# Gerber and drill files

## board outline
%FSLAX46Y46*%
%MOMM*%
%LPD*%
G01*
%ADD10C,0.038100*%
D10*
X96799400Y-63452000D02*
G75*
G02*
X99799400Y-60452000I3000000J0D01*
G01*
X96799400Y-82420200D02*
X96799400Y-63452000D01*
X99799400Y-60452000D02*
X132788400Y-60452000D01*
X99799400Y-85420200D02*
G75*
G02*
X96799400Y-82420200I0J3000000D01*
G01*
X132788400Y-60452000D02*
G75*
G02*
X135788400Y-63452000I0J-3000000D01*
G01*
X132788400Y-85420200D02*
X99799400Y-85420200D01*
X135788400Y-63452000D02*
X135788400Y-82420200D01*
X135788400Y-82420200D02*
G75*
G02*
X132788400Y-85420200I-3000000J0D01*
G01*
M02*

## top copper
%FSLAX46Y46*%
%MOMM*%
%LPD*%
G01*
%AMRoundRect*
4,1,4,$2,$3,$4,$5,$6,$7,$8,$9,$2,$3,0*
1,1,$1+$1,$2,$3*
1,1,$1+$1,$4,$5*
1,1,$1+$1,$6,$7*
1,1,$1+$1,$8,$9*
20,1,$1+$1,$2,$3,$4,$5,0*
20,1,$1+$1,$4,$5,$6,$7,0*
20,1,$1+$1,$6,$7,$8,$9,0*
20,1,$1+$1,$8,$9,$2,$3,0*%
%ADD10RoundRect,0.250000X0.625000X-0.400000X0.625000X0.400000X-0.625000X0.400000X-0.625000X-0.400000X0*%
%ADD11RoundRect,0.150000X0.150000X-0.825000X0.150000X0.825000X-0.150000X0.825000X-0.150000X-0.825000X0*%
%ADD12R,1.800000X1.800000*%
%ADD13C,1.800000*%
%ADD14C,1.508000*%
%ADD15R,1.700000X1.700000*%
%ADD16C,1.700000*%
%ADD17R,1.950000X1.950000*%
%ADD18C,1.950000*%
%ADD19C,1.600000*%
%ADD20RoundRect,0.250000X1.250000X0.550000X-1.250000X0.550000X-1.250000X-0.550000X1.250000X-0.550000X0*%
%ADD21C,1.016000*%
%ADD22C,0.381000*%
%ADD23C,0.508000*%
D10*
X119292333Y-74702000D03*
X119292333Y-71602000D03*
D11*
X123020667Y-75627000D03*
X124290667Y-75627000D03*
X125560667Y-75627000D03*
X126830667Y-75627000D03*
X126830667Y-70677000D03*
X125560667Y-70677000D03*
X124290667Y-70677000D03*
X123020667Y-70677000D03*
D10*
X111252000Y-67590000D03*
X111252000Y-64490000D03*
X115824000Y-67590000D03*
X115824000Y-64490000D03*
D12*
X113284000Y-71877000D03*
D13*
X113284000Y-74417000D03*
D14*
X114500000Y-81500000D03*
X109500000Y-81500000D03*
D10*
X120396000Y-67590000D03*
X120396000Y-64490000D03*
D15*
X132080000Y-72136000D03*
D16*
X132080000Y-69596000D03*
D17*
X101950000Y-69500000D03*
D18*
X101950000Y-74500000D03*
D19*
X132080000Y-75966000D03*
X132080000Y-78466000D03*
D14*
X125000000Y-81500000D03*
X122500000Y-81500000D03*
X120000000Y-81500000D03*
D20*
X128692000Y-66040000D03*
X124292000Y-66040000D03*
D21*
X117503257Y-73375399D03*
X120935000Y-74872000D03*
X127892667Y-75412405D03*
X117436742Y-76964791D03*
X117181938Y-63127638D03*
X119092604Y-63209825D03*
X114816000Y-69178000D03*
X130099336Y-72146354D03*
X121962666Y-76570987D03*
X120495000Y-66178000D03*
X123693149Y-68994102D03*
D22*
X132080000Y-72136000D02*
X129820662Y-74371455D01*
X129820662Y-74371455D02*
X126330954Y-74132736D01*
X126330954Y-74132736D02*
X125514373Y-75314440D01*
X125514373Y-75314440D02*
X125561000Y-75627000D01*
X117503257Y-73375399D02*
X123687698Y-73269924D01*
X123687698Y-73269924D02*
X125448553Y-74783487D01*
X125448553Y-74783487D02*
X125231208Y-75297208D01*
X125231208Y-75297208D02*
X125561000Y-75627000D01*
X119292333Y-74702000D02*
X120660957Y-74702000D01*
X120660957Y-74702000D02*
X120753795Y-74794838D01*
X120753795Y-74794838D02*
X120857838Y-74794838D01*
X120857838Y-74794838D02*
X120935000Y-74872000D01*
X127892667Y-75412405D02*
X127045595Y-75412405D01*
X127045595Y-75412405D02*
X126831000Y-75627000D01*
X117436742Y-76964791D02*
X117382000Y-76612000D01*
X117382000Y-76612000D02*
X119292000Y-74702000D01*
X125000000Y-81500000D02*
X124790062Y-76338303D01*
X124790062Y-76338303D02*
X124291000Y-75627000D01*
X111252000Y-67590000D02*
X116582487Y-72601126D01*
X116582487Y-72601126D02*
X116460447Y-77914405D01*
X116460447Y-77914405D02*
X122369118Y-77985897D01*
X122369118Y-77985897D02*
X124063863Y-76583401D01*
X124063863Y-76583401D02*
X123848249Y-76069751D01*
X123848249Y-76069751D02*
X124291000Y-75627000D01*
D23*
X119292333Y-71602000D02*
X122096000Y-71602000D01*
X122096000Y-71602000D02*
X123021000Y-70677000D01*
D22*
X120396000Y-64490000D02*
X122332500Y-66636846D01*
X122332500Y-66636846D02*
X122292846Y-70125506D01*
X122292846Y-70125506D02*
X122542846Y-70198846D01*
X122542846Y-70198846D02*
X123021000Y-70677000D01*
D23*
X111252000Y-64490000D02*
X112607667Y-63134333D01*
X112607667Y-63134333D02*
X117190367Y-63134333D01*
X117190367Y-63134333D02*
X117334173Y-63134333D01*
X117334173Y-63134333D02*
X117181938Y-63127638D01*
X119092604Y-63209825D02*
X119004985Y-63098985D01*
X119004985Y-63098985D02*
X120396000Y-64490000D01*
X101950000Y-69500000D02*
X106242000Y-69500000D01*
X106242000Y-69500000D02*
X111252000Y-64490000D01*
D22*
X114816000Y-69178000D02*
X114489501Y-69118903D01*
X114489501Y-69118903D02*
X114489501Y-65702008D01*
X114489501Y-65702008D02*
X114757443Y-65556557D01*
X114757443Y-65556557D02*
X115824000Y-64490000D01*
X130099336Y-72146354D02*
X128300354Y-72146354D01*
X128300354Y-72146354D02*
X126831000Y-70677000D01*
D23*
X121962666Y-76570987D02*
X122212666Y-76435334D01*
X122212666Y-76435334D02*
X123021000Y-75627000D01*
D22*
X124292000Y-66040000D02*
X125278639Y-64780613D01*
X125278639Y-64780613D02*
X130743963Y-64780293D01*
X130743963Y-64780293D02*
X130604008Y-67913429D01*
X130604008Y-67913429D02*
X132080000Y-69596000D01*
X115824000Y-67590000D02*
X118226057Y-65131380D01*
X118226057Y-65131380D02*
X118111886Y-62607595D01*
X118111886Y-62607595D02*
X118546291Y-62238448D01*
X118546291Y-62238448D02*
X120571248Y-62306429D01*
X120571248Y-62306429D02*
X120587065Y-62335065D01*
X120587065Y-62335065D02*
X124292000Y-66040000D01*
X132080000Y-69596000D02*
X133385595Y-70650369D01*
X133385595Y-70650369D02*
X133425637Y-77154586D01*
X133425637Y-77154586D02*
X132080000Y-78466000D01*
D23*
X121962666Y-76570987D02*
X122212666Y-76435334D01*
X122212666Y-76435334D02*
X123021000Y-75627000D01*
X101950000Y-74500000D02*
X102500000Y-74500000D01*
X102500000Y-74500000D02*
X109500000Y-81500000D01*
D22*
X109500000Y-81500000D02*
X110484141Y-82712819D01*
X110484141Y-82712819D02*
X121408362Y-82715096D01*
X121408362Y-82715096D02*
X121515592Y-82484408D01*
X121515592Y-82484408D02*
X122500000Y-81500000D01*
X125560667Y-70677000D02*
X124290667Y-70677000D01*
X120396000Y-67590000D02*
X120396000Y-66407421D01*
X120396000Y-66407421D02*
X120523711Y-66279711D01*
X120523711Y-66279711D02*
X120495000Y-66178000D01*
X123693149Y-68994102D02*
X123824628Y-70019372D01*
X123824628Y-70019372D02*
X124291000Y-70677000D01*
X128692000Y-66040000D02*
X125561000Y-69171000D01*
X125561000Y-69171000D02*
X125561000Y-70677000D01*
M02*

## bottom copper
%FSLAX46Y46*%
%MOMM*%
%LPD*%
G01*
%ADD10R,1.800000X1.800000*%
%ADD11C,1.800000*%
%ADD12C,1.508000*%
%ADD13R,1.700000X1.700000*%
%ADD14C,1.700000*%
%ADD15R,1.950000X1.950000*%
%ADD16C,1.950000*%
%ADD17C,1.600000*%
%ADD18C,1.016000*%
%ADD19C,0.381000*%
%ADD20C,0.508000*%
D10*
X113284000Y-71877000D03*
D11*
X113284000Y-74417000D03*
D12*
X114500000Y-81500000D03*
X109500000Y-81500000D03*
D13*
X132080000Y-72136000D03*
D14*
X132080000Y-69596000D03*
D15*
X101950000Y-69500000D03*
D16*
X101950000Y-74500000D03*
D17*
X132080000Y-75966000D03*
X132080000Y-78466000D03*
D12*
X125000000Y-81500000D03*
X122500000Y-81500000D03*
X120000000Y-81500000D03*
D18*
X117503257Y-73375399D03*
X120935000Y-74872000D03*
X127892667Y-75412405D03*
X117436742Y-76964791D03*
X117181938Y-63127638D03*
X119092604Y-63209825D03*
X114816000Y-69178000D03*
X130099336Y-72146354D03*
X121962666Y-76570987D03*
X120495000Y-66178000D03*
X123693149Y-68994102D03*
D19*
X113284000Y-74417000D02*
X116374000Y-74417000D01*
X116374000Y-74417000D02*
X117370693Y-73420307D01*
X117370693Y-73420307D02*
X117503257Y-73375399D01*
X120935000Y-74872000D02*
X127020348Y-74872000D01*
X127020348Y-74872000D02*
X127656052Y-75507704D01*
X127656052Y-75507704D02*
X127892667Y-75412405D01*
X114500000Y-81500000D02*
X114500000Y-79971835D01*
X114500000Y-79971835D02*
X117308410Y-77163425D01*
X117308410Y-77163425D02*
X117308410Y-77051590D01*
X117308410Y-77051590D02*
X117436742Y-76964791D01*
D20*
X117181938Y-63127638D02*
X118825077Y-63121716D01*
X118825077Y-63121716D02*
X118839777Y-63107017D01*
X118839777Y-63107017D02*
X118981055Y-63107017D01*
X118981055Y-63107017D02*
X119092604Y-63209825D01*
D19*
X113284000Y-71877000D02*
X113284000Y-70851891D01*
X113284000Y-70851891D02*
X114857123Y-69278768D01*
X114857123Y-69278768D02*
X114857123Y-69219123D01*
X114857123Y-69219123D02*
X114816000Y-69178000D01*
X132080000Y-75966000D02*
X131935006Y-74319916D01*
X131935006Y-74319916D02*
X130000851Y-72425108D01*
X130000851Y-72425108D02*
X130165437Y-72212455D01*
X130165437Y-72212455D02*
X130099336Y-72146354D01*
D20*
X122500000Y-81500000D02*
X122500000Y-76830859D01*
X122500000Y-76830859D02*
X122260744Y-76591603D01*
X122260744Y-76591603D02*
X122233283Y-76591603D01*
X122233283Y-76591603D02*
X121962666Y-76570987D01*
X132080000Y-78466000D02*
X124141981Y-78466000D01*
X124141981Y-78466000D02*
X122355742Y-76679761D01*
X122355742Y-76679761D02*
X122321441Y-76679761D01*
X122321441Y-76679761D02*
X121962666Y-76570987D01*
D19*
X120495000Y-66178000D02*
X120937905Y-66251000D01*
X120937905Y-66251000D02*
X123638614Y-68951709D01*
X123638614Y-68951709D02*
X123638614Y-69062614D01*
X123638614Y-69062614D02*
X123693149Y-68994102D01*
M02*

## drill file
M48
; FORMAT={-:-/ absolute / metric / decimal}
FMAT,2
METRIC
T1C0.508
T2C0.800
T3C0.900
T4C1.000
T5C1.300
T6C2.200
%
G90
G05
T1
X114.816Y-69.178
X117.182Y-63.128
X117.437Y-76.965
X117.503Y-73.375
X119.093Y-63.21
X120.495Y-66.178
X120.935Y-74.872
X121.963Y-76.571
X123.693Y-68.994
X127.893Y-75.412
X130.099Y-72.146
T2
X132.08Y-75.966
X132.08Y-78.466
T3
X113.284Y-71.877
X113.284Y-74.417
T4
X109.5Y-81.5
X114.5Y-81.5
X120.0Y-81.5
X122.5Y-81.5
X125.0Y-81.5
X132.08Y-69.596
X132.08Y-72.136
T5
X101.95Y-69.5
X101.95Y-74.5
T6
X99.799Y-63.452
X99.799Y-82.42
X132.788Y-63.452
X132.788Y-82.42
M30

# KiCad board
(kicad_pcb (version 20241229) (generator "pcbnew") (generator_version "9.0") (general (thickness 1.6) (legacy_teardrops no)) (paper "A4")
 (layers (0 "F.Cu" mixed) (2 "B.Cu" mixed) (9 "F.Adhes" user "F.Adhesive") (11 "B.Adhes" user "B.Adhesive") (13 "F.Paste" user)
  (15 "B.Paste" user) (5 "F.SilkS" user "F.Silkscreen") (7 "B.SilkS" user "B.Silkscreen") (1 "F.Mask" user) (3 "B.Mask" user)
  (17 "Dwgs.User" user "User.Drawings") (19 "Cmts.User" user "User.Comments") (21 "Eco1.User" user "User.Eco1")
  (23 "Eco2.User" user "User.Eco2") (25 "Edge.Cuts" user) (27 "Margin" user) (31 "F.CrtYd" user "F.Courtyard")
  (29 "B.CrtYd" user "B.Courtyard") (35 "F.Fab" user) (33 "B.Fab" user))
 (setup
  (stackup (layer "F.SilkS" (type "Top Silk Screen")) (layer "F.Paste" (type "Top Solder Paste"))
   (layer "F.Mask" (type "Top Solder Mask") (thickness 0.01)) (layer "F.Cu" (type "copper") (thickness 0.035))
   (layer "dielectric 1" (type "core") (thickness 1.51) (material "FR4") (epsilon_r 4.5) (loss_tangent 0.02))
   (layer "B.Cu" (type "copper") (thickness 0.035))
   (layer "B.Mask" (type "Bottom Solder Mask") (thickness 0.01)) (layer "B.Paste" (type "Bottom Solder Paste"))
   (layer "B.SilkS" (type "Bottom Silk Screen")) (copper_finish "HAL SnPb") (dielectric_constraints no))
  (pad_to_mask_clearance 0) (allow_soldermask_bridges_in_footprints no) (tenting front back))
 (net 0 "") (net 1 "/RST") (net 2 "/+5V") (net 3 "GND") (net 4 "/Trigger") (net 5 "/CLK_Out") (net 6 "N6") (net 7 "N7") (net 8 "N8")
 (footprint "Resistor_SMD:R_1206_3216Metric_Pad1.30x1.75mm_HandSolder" (layer "F.Cu") (at 119.292333 73.152 90)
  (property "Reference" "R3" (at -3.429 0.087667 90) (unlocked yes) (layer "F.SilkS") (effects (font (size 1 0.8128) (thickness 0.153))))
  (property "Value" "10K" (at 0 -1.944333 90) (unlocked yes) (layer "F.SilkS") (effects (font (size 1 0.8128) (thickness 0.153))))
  (pad "1" smd roundrect (at -1.55 0 90) (size 1.3 1.75) (layers "F.Cu" "F.Mask" "F.Paste") (roundrect_rratio 0.192308) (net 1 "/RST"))
  (pad "2" smd roundrect (at 1.55 0 90) (size 1.3 1.75) (layers "F.Cu" "F.Mask" "F.Paste") (roundrect_rratio 0.192308) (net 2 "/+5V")))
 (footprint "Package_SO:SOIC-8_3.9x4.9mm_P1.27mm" (layer "F.Cu") (at 124.925667 73.152 90)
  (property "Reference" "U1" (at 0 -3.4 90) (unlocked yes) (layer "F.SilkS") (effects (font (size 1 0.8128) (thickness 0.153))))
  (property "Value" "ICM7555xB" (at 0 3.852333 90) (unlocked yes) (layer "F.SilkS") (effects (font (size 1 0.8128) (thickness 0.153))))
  (pad "1" smd roundrect (at -2.475 -1.905 90) (size 1.95 0.6) (layers "F.Cu" "F.Mask" "F.Paste") (roundrect_rratio 0.25) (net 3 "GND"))
  (pad "2" smd roundrect (at -2.475 -0.635 90) (size 1.95 0.6) (layers "F.Cu" "F.Mask" "F.Paste") (roundrect_rratio 0.25) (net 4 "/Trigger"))
  (pad "3" smd roundrect (at -2.475 0.635 90) (size 1.95 0.6) (layers "F.Cu" "F.Mask" "F.Paste") (roundrect_rratio 0.25) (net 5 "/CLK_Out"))
  (pad "4" smd roundrect (at -2.475 1.905 90) (size 1.95 0.6) (layers "F.Cu" "F.Mask" "F.Paste") (roundrect_rratio 0.25) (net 1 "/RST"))
  (pad "5" smd roundrect (at 2.475 1.905 90) (size 1.95 0.6) (layers "F.Cu" "F.Mask" "F.Paste") (roundrect_rratio 0.25) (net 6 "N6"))
  (pad "6" smd roundrect (at 2.475 0.635 90) (size 1.95 0.6) (layers "F.Cu" "F.Mask" "F.Paste") (roundrect_rratio 0.25) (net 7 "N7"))
  (pad "7" smd roundrect (at 2.475 -0.635 90) (size 1.95 0.6) (layers "F.Cu" "F.Mask" "F.Paste") (roundrect_rratio 0.25) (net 7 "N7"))
  (pad "8" smd roundrect (at 2.475 -1.905 90) (size 1.95 0.6) (layers "F.Cu" "F.Mask" "F.Paste") (roundrect_rratio 0.25) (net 2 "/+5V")))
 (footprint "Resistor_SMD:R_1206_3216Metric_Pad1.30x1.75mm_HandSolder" (layer "F.Cu") (at 111.252 66.04 90)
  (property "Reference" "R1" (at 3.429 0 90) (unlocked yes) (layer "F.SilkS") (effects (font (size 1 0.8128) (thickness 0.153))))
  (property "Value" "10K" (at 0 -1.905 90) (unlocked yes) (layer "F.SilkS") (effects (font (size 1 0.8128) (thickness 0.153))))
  (pad "1" smd roundrect (at -1.55 0 90) (size 1.3 1.75) (layers "F.Cu" "F.Mask" "F.Paste") (roundrect_rratio 0.192308) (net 4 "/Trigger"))
  (pad "2" smd roundrect (at 1.55 0 90) (size 1.3 1.75) (layers "F.Cu" "F.Mask" "F.Paste") (roundrect_rratio 0.192308) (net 2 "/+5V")))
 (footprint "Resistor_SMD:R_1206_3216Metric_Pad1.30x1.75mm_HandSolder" (layer "F.Cu") (at 115.824 66.04 90)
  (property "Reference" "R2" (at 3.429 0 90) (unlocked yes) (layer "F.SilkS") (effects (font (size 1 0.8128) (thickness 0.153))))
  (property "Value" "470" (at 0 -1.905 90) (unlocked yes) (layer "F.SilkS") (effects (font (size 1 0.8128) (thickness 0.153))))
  (pad "1" smd roundrect (at -1.55 0 90) (size 1.3 1.75) (layers "F.Cu" "F.Mask" "F.Paste") (roundrect_rratio 0.192308) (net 3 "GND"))
  (pad "2" smd roundrect (at 1.55 0 90) (size 1.3 1.75) (layers "F.Cu" "F.Mask" "F.Paste") (roundrect_rratio 0.192308) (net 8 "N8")))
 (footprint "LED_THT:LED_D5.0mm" (layer "F.Cu") (at 113.284 71.877 -90)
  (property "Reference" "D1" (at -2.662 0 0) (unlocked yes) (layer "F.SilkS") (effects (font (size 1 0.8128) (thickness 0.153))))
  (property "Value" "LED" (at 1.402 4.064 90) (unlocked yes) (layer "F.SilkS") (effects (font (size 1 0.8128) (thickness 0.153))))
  (pad "1" thru_hole rect (at 0 0 270) (size 1.8 1.8) (drill 0.9) (layers "*.Cu" "*.Mask") (remove_unused_layers no) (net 8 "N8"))
  (pad "2" thru_hole circle (at 2.54 0 270) (size 1.8 1.8) (drill 0.9) (layers "*.Cu" "*.Mask") (remove_unused_layers no) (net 5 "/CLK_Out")))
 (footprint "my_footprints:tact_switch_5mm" (layer "F.Cu") (at 112 81.5 180)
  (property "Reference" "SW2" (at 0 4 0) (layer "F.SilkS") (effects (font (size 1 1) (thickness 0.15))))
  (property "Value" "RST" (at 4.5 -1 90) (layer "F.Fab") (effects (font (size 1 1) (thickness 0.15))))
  (pad "1" thru_hole circle (at -2.5 0 180) (size 1.508 1.508) (drill 1) (layers "*.Cu" "*.Mask") (remove_unused_layers no) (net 1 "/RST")
   (solder_mask_margin 0.102))
  (pad "2" thru_hole circle (at 2.5 0 180) (size 1.508 1.508) (drill 1) (layers "*.Cu" "*.Mask") (remove_unused_layers no) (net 3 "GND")
   (solder_mask_margin 0.102)))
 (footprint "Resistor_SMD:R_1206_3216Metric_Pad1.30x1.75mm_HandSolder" (layer "F.Cu") (at 120.396 66.04 90)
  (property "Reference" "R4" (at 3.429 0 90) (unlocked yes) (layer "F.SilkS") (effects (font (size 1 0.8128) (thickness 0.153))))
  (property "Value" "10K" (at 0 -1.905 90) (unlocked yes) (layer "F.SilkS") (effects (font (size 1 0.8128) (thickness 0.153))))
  (pad "1" smd roundrect (at -1.55 0 90) (size 1.3 1.75) (layers "F.Cu" "F.Mask" "F.Paste") (roundrect_rratio 0.192308) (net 7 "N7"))
  (pad "2" smd roundrect (at 1.55 0 90) (size 1.3 1.75) (layers "F.Cu" "F.Mask" "F.Paste") (roundrect_rratio 0.192308) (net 2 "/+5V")))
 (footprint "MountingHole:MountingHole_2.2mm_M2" (layer "F.Cu") (at 99.7994 63.452)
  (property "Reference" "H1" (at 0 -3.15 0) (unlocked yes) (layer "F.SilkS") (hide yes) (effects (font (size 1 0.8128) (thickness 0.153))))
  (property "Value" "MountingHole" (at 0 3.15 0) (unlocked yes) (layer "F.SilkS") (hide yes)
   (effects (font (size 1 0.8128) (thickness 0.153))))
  (pad "" np_thru_hole circle (at 0 0) (size 2.2 2.2) (drill 2.2) (layers "*.Cu" "*.Mask")))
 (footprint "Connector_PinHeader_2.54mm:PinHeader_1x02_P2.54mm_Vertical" (layer "F.Cu") (at 132.08 72.136 180)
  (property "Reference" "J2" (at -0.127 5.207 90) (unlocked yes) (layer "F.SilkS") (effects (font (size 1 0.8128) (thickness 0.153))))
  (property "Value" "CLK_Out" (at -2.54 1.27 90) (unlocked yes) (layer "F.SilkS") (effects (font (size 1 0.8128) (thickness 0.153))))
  (pad "1" thru_hole rect (at 0 0 180) (size 1.7 1.7) (drill 1) (layers "*.Cu" "*.Mask") (remove_unused_layers no) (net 5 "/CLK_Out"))
  (pad "2" thru_hole circle (at 0 2.54 180) (size 1.7 1.7) (drill 1) (layers "*.Cu" "*.Mask") (remove_unused_layers no) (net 3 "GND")))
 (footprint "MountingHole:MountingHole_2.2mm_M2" (layer "F.Cu") (at 132.7884 82.4202)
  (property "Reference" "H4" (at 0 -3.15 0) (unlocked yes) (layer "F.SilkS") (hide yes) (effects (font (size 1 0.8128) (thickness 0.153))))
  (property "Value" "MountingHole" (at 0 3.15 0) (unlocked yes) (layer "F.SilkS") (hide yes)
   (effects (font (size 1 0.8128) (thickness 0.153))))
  (pad "" np_thru_hole circle (at 0 0) (size 2.2 2.2) (drill 2.2) (layers "*.Cu" "*.Mask")))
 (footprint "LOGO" (layer "F.Cu") (at 105.5 63.5)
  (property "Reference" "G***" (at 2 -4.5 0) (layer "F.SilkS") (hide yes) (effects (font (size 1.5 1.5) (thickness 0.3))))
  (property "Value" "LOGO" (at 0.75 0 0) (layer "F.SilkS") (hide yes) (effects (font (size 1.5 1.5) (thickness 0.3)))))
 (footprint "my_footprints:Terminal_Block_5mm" (layer "F.Cu") (at 101.95 72 -90)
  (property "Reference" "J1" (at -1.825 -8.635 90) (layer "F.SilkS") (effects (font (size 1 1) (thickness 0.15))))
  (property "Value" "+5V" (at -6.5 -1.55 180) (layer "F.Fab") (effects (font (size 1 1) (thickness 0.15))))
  (pad "1" thru_hole rect (at -2.5 0 270) (size 1.95 1.95) (drill 1.3) (layers "*.Cu" "*.Mask") (remove_unused_layers no) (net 2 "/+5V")
   (solder_mask_margin 0.102))
  (pad "2" thru_hole circle (at 2.5 0 270) (size 1.95 1.95) (drill 1.3) (layers "*.Cu" "*.Mask") (remove_unused_layers no) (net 3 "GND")
   (solder_mask_margin 0.102)))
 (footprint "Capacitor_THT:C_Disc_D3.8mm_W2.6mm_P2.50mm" (layer "F.Cu") (at 132.08 75.966 -90)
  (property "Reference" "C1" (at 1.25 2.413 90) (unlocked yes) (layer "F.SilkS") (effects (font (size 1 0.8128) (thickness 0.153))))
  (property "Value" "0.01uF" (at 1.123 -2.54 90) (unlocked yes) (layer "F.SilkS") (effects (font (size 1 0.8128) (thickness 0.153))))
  (pad "1" thru_hole circle (at 0 0 270) (size 1.6 1.6) (drill 0.8) (layers "*.Cu" "*.Mask") (remove_unused_layers no) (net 6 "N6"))
  (pad "2" thru_hole circle (at 2.5 0 270) (size 1.6 1.6) (drill 0.8) (layers "*.Cu" "*.Mask") (remove_unused_layers no) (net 3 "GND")))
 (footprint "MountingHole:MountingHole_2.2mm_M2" (layer "F.Cu") (at 132.7884 63.452)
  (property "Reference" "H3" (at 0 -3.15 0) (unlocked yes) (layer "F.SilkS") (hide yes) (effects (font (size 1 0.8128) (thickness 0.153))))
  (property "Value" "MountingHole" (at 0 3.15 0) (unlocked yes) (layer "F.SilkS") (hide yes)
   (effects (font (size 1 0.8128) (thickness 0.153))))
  (pad "" np_thru_hole circle (at 0 0) (size 2.2 2.2) (drill 2.2) (layers "*.Cu" "*.Mask")))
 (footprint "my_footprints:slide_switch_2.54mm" (layer "F.Cu") (at 122.5 81.5 180)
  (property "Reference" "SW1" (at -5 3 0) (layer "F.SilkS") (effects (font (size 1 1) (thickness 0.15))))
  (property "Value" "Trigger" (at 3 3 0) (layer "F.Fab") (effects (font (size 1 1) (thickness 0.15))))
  (pad "1" thru_hole circle (at -2.5 0 180) (size 1.508 1.508) (drill 1) (layers "*.Cu" "*.Mask") (remove_unused_layers no)
   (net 4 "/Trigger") (solder_mask_margin 0.102))
  (pad "2" thru_hole circle (at 0 0 180) (size 1.508 1.508) (drill 1) (layers "*.Cu" "*.Mask") (remove_unused_layers no) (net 3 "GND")
   (solder_mask_margin 0.102))
  (pad "3" thru_hole circle (at 2.5 0 180) (size 1.508 1.508) (drill 1) (layers "*.Cu" "*.Mask") (remove_unused_layers no)
   (solder_mask_margin 0.102)))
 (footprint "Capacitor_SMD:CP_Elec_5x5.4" (layer "F.Cu") (at 126.492 66.04 180)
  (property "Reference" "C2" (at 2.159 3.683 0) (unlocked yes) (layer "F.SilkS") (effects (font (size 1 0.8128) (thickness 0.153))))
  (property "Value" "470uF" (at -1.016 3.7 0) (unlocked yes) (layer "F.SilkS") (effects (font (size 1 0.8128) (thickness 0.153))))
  (pad "1" smd roundrect (at -2.2 0 180) (size 3 1.6) (layers "F.Cu" "F.Mask" "F.Paste") (roundrect_rratio 0.15625) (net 7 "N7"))
  (pad "2" smd roundrect (at 2.2 0 180) (size 3 1.6) (layers "F.Cu" "F.Mask" "F.Paste") (roundrect_rratio 0.15625) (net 3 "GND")))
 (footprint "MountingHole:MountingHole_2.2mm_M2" (layer "F.Cu") (at 99.7994 82.4202)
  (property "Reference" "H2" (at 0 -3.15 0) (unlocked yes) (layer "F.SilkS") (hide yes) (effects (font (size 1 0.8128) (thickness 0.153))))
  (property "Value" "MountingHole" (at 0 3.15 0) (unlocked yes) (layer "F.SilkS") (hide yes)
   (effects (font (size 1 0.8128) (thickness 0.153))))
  (pad "" np_thru_hole circle (at 0 0) (size 2.2 2.2) (drill 2.2) (layers "*.Cu" "*.Mask")))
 (gr_arc (start 96.7994 63.452) (mid 97.67808 61.33068) (end 99.7994 60.452) (stroke (width 0.0381) (type default)) (layer "Edge.Cuts"))
 (gr_line (start 96.7994 82.4202) (end 96.7994 63.452) (stroke (width 0.0381) (type default)) (layer "Edge.Cuts"))
 (gr_line (start 99.7994 60.452) (end 132.7884 60.452) (stroke (width 0.0381) (type default)) (layer "Edge.Cuts"))
 (gr_arc (start 99.7994 85.4202) (mid 97.67808 84.54152) (end 96.7994 82.4202) (stroke (width 0.0381) (type default)) (layer "Edge.Cuts"))
 (gr_arc (start 132.7884 60.452) (mid 134.90972 61.33068) (end 135.7884 63.452) (stroke (width 0.0381) (type default)) (layer "Edge.Cuts"))
 (gr_line (start 132.7884 85.4202) (end 99.7994 85.4202) (stroke (width 0.0381) (type default)) (layer "Edge.Cuts"))
 (gr_line (start 135.7884 63.452) (end 135.7884 82.4202) (stroke (width 0.0381) (type default)) (layer "Edge.Cuts"))
 (gr_arc (start 135.7884 82.4202) (mid 134.90972 84.54152) (end 132.7884 85.4202) (stroke (width 0.0381) (type default)) (layer "Edge.Cuts"))
 (segment (start 132.080000 72.136000) (end 129.820662 74.371455) (width 0.381000) (layer "F.Cu") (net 5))
 (segment (start 129.820662 74.371455) (end 126.330954 74.132736) (width 0.381000) (layer "F.Cu") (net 5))
 (segment (start 126.330954 74.132736) (end 125.514373 75.314440) (width 0.381000) (layer "F.Cu") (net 5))
 (segment (start 125.514373 75.314440) (end 125.561000 75.627000) (width 0.381000) (layer "F.Cu") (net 5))
 (segment (start 113.284000 74.417000) (end 116.374000 74.417000) (width 0.381000) (layer "B.Cu") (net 5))
 (segment (start 116.374000 74.417000) (end 117.370693 73.420307) (width 0.381000) (layer "B.Cu") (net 5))
 (segment (start 117.370693 73.420307) (end 117.503257 73.375399) (width 0.381000) (layer "B.Cu") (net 5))
 (segment (start 117.503257 73.375399) (end 123.687698 73.269924) (width 0.381000) (layer "F.Cu") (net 5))
 (segment (start 123.687698 73.269924) (end 125.448553 74.783487) (width 0.381000) (layer "F.Cu") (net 5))
 (segment (start 125.448553 74.783487) (end 125.231208 75.297208) (width 0.381000) (layer "F.Cu") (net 5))
 (segment (start 125.231208 75.297208) (end 125.561000 75.627000) (width 0.381000) (layer "F.Cu") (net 5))
 (segment (start 119.292333 74.702000) (end 120.660957 74.702000) (width 0.381000) (layer "F.Cu") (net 1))
 (segment (start 120.660957 74.702000) (end 120.753795 74.794838) (width 0.381000) (layer "F.Cu") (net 1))
 (segment (start 120.753795 74.794838) (end 120.857838 74.794838) (width 0.381000) (layer "F.Cu") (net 1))
 (segment (start 120.857838 74.794838) (end 120.935000 74.872000) (width 0.381000) (layer "F.Cu") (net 1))
 (segment (start 120.935000 74.872000) (end 127.020348 74.872000) (width 0.381000) (layer "B.Cu") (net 1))
 (segment (start 127.020348 74.872000) (end 127.656052 75.507704) (width 0.381000) (layer "B.Cu") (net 1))
 (segment (start 127.656052 75.507704) (end 127.892667 75.412405) (width 0.381000) (layer "B.Cu") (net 1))
 (segment (start 127.892667 75.412405) (end 127.045595 75.412405) (width 0.381000) (layer "F.Cu") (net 1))
 (segment (start 127.045595 75.412405) (end 126.831000 75.627000) (width 0.381000) (layer "F.Cu") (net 1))
 (segment (start 114.500000 81.500000) (end 114.500000 79.971835) (width 0.381000) (layer "B.Cu") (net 1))
 (segment (start 114.500000 79.971835) (end 117.308410 77.163425) (width 0.381000) (layer "B.Cu") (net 1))
 (segment (start 117.308410 77.163425) (end 117.308410 77.051590) (width 0.381000) (layer "B.Cu") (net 1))
 (segment (start 117.308410 77.051590) (end 117.436742 76.964791) (width 0.381000) (layer "B.Cu") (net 1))
 (segment (start 117.436742 76.964791) (end 117.382000 76.612000) (width 0.381000) (layer "F.Cu") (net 1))
 (segment (start 117.382000 76.612000) (end 119.292000 74.702000) (width 0.381000) (layer "F.Cu") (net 1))
 (segment (start 125.000000 81.500000) (end 124.790062 76.338303) (width 0.381000) (layer "F.Cu") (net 4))
 (segment (start 124.790062 76.338303) (end 124.291000 75.627000) (width 0.381000) (layer "F.Cu") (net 4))
 (segment (start 111.252000 67.590000) (end 116.582487 72.601126) (width 0.381000) (layer "F.Cu") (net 4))
 (segment (start 116.582487 72.601126) (end 116.460447 77.914405) (width 0.381000) (layer "F.Cu") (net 4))
 (segment (start 116.460447 77.914405) (end 122.369118 77.985897) (width 0.381000) (layer "F.Cu") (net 4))
 (segment (start 122.369118 77.985897) (end 124.063863 76.583401) (width 0.381000) (layer "F.Cu") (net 4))
 (segment (start 124.063863 76.583401) (end 123.848249 76.069751) (width 0.381000) (layer "F.Cu") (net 4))
 (segment (start 123.848249 76.069751) (end 124.291000 75.627000) (width 0.381000) (layer "F.Cu") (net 4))
 (segment (start 119.292333 71.602000) (end 122.096000 71.602000) (width 0.508000) (layer "F.Cu") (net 2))
 (segment (start 122.096000 71.602000) (end 123.021000 70.677000) (width 0.508000) (layer "F.Cu") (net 2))
 (segment (start 120.396000 64.490000) (end 122.332500 66.636846) (width 0.381000) (layer "F.Cu") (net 2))
 (segment (start 122.332500 66.636846) (end 122.292846 70.125506) (width 0.381000) (layer "F.Cu") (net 2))
 (segment (start 122.292846 70.125506) (end 122.542846 70.198846) (width 0.381000) (layer "F.Cu") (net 2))
 (segment (start 122.542846 70.198846) (end 123.021000 70.677000) (width 0.381000) (layer "F.Cu") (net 2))
 (segment (start 111.252000 64.490000) (end 112.607667 63.134333) (width 0.508000) (layer "F.Cu") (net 2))
 (segment (start 112.607667 63.134333) (end 117.190367 63.134333) (width 0.508000) (layer "F.Cu") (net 2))
 (segment (start 117.190367 63.134333) (end 117.334173 63.134333) (width 0.508000) (layer "F.Cu") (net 2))
 (segment (start 117.334173 63.134333) (end 117.181938 63.127638) (width 0.508000) (layer "F.Cu") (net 2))
 (segment (start 117.181938 63.127638) (end 118.825077 63.121716) (width 0.508000) (layer "B.Cu") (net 2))
 (segment (start 118.825077 63.121716) (end 118.839777 63.107017) (width 0.508000) (layer "B.Cu") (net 2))
 (segment (start 118.839777 63.107017) (end 118.981055 63.107017) (width 0.508000) (layer "B.Cu") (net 2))
 (segment (start 118.981055 63.107017) (end 119.092604 63.209825) (width 0.508000) (layer "B.Cu") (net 2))
 (segment (start 119.092604 63.209825) (end 119.004985 63.098985) (width 0.508000) (layer "F.Cu") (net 2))
 (segment (start 119.004985 63.098985) (end 120.396000 64.490000) (width 0.508000) (layer "F.Cu") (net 2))
 (segment (start 101.950000 69.500000) (end 106.242000 69.500000) (width 0.508000) (layer "F.Cu") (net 2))
 (segment (start 106.242000 69.500000) (end 111.252000 64.490000) (width 0.508000) (layer "F.Cu") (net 2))
 (segment (start 113.284000 71.877000) (end 113.284000 70.851891) (width 0.381000) (layer "B.Cu") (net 8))
 (segment (start 113.284000 70.851891) (end 114.857123 69.278768) (width 0.381000) (layer "B.Cu") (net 8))
 (segment (start 114.857123 69.278768) (end 114.857123 69.219123) (width 0.381000) (layer "B.Cu") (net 8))
 (segment (start 114.857123 69.219123) (end 114.816000 69.178000) (width 0.381000) (layer "B.Cu") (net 8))
 (segment (start 114.816000 69.178000) (end 114.489501 69.118903) (width 0.381000) (layer "F.Cu") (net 8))
 (segment (start 114.489501 69.118903) (end 114.489501 65.702008) (width 0.381000) (layer "F.Cu") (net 8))
 (segment (start 114.489501 65.702008) (end 114.757443 65.556557) (width 0.381000) (layer "F.Cu") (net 8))
 (segment (start 114.757443 65.556557) (end 115.824000 64.490000) (width 0.381000) (layer "F.Cu") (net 8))
 (segment (start 132.080000 75.966000) (end 131.935006 74.319916) (width 0.381000) (layer "B.Cu") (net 6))
 (segment (start 131.935006 74.319916) (end 130.000851 72.425108) (width 0.381000) (layer "B.Cu") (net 6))
 (segment (start 130.000851 72.425108) (end 130.165437 72.212455) (width 0.381000) (layer "B.Cu") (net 6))
 (segment (start 130.165437 72.212455) (end 130.099336 72.146354) (width 0.381000) (layer "B.Cu") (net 6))
 (segment (start 130.099336 72.146354) (end 128.300354 72.146354) (width 0.381000) (layer "F.Cu") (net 6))
 (segment (start 128.300354 72.146354) (end 126.831000 70.677000) (width 0.381000) (layer "F.Cu") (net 6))
 (segment (start 122.500000 81.500000) (end 122.500000 76.830859) (width 0.508000) (layer "B.Cu") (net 3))
 (segment (start 122.500000 76.830859) (end 122.260744 76.591603) (width 0.508000) (layer "B.Cu") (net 3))
 (segment (start 122.260744 76.591603) (end 122.233283 76.591603) (width 0.508000) (layer "B.Cu") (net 3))
 (segment (start 122.233283 76.591603) (end 121.962666 76.570987) (width 0.508000) (layer "B.Cu") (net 3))
 (segment (start 121.962666 76.570987) (end 122.212666 76.435334) (width 0.508000) (layer "F.Cu") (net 3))
 (segment (start 122.212666 76.435334) (end 123.021000 75.627000) (width 0.508000) (layer "F.Cu") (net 3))
 (segment (start 124.292000 66.040000) (end 125.278639 64.780613) (width 0.381000) (layer "F.Cu") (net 3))
 (segment (start 125.278639 64.780613) (end 130.743963 64.780293) (width 0.381000) (layer "F.Cu") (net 3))
 (segment (start 130.743963 64.780293) (end 130.604008 67.913429) (width 0.381000) (layer "F.Cu") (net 3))
 (segment (start 130.604008 67.913429) (end 132.080000 69.596000) (width 0.381000) (layer "F.Cu") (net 3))
 (segment (start 115.824000 67.590000) (end 118.226057 65.131380) (width 0.381000) (layer "F.Cu") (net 3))
 (segment (start 118.226057 65.131380) (end 118.111886 62.607595) (width 0.381000) (layer "F.Cu") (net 3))
 (segment (start 118.111886 62.607595) (end 118.546291 62.238448) (width 0.381000) (layer "F.Cu") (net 3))
 (segment (start 118.546291 62.238448) (end 120.571248 62.306429) (width 0.381000) (layer "F.Cu") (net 3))
 (segment (start 120.571248 62.306429) (end 120.587065 62.335065) (width 0.381000) (layer "F.Cu") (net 3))
 (segment (start 120.587065 62.335065) (end 124.292000 66.040000) (width 0.381000) (layer "F.Cu") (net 3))
 (segment (start 132.080000 69.596000) (end 133.385595 70.650369) (width 0.381000) (layer "F.Cu") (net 3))
 (segment (start 133.385595 70.650369) (end 133.425637 77.154586) (width 0.381000) (layer "F.Cu") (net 3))
 (segment (start 133.425637 77.154586) (end 132.080000 78.466000) (width 0.381000) (layer "F.Cu") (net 3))
 (segment (start 132.080000 78.466000) (end 124.141981 78.466000) (width 0.508000) (layer "B.Cu") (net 3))
 (segment (start 124.141981 78.466000) (end 122.355742 76.679761) (width 0.508000) (layer "B.Cu") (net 3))
 (segment (start 122.355742 76.679761) (end 122.321441 76.679761) (width 0.508000) (layer "B.Cu") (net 3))
 (segment (start 122.321441 76.679761) (end 121.962666 76.570987) (width 0.508000) (layer "B.Cu") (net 3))
 (segment (start 121.962666 76.570987) (end 122.212666 76.435334) (width 0.508000) (layer "F.Cu") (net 3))
 (segment (start 122.212666 76.435334) (end 123.021000 75.627000) (width 0.508000) (layer "F.Cu") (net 3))
 (segment (start 101.950000 74.500000) (end 102.500000 74.500000) (width 0.508000) (layer "F.Cu") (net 3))
 (segment (start 102.500000 74.500000) (end 109.500000 81.500000) (width 0.508000) (layer "F.Cu") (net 3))
 (segment (start 109.500000 81.500000) (end 110.484141 82.712819) (width 0.381000) (layer "F.Cu") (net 3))
 (segment (start 110.484141 82.712819) (end 121.408362 82.715096) (width 0.381000) (layer "F.Cu") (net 3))
 (segment (start 121.408362 82.715096) (end 121.515592 82.484408) (width 0.381000) (layer "F.Cu") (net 3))
 (segment (start 121.515592 82.484408) (end 122.500000 81.500000) (width 0.381000) (layer "F.Cu") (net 3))
 (segment (start 125.560667 70.677000) (end 124.290667 70.677000) (width 0.381000) (layer "F.Cu") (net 7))
 (segment (start 120.396000 67.590000) (end 120.396000 66.407421) (width 0.381000) (layer "F.Cu") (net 7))
 (segment (start 120.396000 66.407421) (end 120.523711 66.279711) (width 0.381000) (layer "F.Cu") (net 7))
 (segment (start 120.523711 66.279711) (end 120.495000 66.178000) (width 0.381000) (layer "F.Cu") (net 7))
 (segment (start 120.495000 66.178000) (end 120.937905 66.251000) (width 0.381000) (layer "B.Cu") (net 7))
 (segment (start 120.937905 66.251000) (end 123.638614 68.951709) (width 0.381000) (layer "B.Cu") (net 7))
 (segment (start 123.638614 68.951709) (end 123.638614 69.062614) (width 0.381000) (layer "B.Cu") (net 7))
 (segment (start 123.638614 69.062614) (end 123.693149 68.994102) (width 0.381000) (layer "B.Cu") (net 7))
 (segment (start 123.693149 68.994102) (end 123.824628 70.019372) (width 0.381000) (layer "F.Cu") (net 7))
 (segment (start 123.824628 70.019372) (end 124.291000 70.677000) (width 0.381000) (layer "F.Cu") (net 7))
 (segment (start 128.692000 66.040000) (end 125.561000 69.171000) (width 0.381000) (layer "F.Cu") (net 7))
 (segment (start 125.561000 69.171000) (end 125.561000 70.677000) (width 0.381000) (layer "F.Cu") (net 7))
 (via (at 117.503257 73.375399) (size 1.016000) (drill 0.508000) (layers "F.Cu" "B.Cu") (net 5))
 (via (at 120.935000 74.872000) (size 1.016000) (drill 0.508000) (layers "F.Cu" "B.Cu") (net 1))
 (via (at 127.892667 75.412405) (size 1.016000) (drill 0.508000) (layers "F.Cu" "B.Cu") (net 1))
 (via (at 117.436742 76.964791) (size 1.016000) (drill 0.508000) (layers "F.Cu" "B.Cu") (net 1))
 (via (at 117.181938 63.127638) (size 1.016000) (drill 0.508000) (layers "F.Cu" "B.Cu") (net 2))
 (via (at 119.092604 63.209825) (size 1.016000) (drill 0.508000) (layers "F.Cu" "B.Cu") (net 2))
 (via (at 114.816000 69.178000) (size 1.016000) (drill 0.508000) (layers "F.Cu" "B.Cu") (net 8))
 (via (at 130.099336 72.146354) (size 1.016000) (drill 0.508000) (layers "F.Cu" "B.Cu") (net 6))
 (via (at 121.962666 76.570987) (size 1.016000) (drill 0.508000) (layers "F.Cu" "B.Cu") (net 3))
 (via (at 120.495000 66.178000) (size 1.016000) (drill 0.508000) (layers "F.Cu" "B.Cu") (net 7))
 (via (at 123.693149 68.994102) (size 1.016000) (drill 0.508000) (layers "F.Cu" "B.Cu") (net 7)))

